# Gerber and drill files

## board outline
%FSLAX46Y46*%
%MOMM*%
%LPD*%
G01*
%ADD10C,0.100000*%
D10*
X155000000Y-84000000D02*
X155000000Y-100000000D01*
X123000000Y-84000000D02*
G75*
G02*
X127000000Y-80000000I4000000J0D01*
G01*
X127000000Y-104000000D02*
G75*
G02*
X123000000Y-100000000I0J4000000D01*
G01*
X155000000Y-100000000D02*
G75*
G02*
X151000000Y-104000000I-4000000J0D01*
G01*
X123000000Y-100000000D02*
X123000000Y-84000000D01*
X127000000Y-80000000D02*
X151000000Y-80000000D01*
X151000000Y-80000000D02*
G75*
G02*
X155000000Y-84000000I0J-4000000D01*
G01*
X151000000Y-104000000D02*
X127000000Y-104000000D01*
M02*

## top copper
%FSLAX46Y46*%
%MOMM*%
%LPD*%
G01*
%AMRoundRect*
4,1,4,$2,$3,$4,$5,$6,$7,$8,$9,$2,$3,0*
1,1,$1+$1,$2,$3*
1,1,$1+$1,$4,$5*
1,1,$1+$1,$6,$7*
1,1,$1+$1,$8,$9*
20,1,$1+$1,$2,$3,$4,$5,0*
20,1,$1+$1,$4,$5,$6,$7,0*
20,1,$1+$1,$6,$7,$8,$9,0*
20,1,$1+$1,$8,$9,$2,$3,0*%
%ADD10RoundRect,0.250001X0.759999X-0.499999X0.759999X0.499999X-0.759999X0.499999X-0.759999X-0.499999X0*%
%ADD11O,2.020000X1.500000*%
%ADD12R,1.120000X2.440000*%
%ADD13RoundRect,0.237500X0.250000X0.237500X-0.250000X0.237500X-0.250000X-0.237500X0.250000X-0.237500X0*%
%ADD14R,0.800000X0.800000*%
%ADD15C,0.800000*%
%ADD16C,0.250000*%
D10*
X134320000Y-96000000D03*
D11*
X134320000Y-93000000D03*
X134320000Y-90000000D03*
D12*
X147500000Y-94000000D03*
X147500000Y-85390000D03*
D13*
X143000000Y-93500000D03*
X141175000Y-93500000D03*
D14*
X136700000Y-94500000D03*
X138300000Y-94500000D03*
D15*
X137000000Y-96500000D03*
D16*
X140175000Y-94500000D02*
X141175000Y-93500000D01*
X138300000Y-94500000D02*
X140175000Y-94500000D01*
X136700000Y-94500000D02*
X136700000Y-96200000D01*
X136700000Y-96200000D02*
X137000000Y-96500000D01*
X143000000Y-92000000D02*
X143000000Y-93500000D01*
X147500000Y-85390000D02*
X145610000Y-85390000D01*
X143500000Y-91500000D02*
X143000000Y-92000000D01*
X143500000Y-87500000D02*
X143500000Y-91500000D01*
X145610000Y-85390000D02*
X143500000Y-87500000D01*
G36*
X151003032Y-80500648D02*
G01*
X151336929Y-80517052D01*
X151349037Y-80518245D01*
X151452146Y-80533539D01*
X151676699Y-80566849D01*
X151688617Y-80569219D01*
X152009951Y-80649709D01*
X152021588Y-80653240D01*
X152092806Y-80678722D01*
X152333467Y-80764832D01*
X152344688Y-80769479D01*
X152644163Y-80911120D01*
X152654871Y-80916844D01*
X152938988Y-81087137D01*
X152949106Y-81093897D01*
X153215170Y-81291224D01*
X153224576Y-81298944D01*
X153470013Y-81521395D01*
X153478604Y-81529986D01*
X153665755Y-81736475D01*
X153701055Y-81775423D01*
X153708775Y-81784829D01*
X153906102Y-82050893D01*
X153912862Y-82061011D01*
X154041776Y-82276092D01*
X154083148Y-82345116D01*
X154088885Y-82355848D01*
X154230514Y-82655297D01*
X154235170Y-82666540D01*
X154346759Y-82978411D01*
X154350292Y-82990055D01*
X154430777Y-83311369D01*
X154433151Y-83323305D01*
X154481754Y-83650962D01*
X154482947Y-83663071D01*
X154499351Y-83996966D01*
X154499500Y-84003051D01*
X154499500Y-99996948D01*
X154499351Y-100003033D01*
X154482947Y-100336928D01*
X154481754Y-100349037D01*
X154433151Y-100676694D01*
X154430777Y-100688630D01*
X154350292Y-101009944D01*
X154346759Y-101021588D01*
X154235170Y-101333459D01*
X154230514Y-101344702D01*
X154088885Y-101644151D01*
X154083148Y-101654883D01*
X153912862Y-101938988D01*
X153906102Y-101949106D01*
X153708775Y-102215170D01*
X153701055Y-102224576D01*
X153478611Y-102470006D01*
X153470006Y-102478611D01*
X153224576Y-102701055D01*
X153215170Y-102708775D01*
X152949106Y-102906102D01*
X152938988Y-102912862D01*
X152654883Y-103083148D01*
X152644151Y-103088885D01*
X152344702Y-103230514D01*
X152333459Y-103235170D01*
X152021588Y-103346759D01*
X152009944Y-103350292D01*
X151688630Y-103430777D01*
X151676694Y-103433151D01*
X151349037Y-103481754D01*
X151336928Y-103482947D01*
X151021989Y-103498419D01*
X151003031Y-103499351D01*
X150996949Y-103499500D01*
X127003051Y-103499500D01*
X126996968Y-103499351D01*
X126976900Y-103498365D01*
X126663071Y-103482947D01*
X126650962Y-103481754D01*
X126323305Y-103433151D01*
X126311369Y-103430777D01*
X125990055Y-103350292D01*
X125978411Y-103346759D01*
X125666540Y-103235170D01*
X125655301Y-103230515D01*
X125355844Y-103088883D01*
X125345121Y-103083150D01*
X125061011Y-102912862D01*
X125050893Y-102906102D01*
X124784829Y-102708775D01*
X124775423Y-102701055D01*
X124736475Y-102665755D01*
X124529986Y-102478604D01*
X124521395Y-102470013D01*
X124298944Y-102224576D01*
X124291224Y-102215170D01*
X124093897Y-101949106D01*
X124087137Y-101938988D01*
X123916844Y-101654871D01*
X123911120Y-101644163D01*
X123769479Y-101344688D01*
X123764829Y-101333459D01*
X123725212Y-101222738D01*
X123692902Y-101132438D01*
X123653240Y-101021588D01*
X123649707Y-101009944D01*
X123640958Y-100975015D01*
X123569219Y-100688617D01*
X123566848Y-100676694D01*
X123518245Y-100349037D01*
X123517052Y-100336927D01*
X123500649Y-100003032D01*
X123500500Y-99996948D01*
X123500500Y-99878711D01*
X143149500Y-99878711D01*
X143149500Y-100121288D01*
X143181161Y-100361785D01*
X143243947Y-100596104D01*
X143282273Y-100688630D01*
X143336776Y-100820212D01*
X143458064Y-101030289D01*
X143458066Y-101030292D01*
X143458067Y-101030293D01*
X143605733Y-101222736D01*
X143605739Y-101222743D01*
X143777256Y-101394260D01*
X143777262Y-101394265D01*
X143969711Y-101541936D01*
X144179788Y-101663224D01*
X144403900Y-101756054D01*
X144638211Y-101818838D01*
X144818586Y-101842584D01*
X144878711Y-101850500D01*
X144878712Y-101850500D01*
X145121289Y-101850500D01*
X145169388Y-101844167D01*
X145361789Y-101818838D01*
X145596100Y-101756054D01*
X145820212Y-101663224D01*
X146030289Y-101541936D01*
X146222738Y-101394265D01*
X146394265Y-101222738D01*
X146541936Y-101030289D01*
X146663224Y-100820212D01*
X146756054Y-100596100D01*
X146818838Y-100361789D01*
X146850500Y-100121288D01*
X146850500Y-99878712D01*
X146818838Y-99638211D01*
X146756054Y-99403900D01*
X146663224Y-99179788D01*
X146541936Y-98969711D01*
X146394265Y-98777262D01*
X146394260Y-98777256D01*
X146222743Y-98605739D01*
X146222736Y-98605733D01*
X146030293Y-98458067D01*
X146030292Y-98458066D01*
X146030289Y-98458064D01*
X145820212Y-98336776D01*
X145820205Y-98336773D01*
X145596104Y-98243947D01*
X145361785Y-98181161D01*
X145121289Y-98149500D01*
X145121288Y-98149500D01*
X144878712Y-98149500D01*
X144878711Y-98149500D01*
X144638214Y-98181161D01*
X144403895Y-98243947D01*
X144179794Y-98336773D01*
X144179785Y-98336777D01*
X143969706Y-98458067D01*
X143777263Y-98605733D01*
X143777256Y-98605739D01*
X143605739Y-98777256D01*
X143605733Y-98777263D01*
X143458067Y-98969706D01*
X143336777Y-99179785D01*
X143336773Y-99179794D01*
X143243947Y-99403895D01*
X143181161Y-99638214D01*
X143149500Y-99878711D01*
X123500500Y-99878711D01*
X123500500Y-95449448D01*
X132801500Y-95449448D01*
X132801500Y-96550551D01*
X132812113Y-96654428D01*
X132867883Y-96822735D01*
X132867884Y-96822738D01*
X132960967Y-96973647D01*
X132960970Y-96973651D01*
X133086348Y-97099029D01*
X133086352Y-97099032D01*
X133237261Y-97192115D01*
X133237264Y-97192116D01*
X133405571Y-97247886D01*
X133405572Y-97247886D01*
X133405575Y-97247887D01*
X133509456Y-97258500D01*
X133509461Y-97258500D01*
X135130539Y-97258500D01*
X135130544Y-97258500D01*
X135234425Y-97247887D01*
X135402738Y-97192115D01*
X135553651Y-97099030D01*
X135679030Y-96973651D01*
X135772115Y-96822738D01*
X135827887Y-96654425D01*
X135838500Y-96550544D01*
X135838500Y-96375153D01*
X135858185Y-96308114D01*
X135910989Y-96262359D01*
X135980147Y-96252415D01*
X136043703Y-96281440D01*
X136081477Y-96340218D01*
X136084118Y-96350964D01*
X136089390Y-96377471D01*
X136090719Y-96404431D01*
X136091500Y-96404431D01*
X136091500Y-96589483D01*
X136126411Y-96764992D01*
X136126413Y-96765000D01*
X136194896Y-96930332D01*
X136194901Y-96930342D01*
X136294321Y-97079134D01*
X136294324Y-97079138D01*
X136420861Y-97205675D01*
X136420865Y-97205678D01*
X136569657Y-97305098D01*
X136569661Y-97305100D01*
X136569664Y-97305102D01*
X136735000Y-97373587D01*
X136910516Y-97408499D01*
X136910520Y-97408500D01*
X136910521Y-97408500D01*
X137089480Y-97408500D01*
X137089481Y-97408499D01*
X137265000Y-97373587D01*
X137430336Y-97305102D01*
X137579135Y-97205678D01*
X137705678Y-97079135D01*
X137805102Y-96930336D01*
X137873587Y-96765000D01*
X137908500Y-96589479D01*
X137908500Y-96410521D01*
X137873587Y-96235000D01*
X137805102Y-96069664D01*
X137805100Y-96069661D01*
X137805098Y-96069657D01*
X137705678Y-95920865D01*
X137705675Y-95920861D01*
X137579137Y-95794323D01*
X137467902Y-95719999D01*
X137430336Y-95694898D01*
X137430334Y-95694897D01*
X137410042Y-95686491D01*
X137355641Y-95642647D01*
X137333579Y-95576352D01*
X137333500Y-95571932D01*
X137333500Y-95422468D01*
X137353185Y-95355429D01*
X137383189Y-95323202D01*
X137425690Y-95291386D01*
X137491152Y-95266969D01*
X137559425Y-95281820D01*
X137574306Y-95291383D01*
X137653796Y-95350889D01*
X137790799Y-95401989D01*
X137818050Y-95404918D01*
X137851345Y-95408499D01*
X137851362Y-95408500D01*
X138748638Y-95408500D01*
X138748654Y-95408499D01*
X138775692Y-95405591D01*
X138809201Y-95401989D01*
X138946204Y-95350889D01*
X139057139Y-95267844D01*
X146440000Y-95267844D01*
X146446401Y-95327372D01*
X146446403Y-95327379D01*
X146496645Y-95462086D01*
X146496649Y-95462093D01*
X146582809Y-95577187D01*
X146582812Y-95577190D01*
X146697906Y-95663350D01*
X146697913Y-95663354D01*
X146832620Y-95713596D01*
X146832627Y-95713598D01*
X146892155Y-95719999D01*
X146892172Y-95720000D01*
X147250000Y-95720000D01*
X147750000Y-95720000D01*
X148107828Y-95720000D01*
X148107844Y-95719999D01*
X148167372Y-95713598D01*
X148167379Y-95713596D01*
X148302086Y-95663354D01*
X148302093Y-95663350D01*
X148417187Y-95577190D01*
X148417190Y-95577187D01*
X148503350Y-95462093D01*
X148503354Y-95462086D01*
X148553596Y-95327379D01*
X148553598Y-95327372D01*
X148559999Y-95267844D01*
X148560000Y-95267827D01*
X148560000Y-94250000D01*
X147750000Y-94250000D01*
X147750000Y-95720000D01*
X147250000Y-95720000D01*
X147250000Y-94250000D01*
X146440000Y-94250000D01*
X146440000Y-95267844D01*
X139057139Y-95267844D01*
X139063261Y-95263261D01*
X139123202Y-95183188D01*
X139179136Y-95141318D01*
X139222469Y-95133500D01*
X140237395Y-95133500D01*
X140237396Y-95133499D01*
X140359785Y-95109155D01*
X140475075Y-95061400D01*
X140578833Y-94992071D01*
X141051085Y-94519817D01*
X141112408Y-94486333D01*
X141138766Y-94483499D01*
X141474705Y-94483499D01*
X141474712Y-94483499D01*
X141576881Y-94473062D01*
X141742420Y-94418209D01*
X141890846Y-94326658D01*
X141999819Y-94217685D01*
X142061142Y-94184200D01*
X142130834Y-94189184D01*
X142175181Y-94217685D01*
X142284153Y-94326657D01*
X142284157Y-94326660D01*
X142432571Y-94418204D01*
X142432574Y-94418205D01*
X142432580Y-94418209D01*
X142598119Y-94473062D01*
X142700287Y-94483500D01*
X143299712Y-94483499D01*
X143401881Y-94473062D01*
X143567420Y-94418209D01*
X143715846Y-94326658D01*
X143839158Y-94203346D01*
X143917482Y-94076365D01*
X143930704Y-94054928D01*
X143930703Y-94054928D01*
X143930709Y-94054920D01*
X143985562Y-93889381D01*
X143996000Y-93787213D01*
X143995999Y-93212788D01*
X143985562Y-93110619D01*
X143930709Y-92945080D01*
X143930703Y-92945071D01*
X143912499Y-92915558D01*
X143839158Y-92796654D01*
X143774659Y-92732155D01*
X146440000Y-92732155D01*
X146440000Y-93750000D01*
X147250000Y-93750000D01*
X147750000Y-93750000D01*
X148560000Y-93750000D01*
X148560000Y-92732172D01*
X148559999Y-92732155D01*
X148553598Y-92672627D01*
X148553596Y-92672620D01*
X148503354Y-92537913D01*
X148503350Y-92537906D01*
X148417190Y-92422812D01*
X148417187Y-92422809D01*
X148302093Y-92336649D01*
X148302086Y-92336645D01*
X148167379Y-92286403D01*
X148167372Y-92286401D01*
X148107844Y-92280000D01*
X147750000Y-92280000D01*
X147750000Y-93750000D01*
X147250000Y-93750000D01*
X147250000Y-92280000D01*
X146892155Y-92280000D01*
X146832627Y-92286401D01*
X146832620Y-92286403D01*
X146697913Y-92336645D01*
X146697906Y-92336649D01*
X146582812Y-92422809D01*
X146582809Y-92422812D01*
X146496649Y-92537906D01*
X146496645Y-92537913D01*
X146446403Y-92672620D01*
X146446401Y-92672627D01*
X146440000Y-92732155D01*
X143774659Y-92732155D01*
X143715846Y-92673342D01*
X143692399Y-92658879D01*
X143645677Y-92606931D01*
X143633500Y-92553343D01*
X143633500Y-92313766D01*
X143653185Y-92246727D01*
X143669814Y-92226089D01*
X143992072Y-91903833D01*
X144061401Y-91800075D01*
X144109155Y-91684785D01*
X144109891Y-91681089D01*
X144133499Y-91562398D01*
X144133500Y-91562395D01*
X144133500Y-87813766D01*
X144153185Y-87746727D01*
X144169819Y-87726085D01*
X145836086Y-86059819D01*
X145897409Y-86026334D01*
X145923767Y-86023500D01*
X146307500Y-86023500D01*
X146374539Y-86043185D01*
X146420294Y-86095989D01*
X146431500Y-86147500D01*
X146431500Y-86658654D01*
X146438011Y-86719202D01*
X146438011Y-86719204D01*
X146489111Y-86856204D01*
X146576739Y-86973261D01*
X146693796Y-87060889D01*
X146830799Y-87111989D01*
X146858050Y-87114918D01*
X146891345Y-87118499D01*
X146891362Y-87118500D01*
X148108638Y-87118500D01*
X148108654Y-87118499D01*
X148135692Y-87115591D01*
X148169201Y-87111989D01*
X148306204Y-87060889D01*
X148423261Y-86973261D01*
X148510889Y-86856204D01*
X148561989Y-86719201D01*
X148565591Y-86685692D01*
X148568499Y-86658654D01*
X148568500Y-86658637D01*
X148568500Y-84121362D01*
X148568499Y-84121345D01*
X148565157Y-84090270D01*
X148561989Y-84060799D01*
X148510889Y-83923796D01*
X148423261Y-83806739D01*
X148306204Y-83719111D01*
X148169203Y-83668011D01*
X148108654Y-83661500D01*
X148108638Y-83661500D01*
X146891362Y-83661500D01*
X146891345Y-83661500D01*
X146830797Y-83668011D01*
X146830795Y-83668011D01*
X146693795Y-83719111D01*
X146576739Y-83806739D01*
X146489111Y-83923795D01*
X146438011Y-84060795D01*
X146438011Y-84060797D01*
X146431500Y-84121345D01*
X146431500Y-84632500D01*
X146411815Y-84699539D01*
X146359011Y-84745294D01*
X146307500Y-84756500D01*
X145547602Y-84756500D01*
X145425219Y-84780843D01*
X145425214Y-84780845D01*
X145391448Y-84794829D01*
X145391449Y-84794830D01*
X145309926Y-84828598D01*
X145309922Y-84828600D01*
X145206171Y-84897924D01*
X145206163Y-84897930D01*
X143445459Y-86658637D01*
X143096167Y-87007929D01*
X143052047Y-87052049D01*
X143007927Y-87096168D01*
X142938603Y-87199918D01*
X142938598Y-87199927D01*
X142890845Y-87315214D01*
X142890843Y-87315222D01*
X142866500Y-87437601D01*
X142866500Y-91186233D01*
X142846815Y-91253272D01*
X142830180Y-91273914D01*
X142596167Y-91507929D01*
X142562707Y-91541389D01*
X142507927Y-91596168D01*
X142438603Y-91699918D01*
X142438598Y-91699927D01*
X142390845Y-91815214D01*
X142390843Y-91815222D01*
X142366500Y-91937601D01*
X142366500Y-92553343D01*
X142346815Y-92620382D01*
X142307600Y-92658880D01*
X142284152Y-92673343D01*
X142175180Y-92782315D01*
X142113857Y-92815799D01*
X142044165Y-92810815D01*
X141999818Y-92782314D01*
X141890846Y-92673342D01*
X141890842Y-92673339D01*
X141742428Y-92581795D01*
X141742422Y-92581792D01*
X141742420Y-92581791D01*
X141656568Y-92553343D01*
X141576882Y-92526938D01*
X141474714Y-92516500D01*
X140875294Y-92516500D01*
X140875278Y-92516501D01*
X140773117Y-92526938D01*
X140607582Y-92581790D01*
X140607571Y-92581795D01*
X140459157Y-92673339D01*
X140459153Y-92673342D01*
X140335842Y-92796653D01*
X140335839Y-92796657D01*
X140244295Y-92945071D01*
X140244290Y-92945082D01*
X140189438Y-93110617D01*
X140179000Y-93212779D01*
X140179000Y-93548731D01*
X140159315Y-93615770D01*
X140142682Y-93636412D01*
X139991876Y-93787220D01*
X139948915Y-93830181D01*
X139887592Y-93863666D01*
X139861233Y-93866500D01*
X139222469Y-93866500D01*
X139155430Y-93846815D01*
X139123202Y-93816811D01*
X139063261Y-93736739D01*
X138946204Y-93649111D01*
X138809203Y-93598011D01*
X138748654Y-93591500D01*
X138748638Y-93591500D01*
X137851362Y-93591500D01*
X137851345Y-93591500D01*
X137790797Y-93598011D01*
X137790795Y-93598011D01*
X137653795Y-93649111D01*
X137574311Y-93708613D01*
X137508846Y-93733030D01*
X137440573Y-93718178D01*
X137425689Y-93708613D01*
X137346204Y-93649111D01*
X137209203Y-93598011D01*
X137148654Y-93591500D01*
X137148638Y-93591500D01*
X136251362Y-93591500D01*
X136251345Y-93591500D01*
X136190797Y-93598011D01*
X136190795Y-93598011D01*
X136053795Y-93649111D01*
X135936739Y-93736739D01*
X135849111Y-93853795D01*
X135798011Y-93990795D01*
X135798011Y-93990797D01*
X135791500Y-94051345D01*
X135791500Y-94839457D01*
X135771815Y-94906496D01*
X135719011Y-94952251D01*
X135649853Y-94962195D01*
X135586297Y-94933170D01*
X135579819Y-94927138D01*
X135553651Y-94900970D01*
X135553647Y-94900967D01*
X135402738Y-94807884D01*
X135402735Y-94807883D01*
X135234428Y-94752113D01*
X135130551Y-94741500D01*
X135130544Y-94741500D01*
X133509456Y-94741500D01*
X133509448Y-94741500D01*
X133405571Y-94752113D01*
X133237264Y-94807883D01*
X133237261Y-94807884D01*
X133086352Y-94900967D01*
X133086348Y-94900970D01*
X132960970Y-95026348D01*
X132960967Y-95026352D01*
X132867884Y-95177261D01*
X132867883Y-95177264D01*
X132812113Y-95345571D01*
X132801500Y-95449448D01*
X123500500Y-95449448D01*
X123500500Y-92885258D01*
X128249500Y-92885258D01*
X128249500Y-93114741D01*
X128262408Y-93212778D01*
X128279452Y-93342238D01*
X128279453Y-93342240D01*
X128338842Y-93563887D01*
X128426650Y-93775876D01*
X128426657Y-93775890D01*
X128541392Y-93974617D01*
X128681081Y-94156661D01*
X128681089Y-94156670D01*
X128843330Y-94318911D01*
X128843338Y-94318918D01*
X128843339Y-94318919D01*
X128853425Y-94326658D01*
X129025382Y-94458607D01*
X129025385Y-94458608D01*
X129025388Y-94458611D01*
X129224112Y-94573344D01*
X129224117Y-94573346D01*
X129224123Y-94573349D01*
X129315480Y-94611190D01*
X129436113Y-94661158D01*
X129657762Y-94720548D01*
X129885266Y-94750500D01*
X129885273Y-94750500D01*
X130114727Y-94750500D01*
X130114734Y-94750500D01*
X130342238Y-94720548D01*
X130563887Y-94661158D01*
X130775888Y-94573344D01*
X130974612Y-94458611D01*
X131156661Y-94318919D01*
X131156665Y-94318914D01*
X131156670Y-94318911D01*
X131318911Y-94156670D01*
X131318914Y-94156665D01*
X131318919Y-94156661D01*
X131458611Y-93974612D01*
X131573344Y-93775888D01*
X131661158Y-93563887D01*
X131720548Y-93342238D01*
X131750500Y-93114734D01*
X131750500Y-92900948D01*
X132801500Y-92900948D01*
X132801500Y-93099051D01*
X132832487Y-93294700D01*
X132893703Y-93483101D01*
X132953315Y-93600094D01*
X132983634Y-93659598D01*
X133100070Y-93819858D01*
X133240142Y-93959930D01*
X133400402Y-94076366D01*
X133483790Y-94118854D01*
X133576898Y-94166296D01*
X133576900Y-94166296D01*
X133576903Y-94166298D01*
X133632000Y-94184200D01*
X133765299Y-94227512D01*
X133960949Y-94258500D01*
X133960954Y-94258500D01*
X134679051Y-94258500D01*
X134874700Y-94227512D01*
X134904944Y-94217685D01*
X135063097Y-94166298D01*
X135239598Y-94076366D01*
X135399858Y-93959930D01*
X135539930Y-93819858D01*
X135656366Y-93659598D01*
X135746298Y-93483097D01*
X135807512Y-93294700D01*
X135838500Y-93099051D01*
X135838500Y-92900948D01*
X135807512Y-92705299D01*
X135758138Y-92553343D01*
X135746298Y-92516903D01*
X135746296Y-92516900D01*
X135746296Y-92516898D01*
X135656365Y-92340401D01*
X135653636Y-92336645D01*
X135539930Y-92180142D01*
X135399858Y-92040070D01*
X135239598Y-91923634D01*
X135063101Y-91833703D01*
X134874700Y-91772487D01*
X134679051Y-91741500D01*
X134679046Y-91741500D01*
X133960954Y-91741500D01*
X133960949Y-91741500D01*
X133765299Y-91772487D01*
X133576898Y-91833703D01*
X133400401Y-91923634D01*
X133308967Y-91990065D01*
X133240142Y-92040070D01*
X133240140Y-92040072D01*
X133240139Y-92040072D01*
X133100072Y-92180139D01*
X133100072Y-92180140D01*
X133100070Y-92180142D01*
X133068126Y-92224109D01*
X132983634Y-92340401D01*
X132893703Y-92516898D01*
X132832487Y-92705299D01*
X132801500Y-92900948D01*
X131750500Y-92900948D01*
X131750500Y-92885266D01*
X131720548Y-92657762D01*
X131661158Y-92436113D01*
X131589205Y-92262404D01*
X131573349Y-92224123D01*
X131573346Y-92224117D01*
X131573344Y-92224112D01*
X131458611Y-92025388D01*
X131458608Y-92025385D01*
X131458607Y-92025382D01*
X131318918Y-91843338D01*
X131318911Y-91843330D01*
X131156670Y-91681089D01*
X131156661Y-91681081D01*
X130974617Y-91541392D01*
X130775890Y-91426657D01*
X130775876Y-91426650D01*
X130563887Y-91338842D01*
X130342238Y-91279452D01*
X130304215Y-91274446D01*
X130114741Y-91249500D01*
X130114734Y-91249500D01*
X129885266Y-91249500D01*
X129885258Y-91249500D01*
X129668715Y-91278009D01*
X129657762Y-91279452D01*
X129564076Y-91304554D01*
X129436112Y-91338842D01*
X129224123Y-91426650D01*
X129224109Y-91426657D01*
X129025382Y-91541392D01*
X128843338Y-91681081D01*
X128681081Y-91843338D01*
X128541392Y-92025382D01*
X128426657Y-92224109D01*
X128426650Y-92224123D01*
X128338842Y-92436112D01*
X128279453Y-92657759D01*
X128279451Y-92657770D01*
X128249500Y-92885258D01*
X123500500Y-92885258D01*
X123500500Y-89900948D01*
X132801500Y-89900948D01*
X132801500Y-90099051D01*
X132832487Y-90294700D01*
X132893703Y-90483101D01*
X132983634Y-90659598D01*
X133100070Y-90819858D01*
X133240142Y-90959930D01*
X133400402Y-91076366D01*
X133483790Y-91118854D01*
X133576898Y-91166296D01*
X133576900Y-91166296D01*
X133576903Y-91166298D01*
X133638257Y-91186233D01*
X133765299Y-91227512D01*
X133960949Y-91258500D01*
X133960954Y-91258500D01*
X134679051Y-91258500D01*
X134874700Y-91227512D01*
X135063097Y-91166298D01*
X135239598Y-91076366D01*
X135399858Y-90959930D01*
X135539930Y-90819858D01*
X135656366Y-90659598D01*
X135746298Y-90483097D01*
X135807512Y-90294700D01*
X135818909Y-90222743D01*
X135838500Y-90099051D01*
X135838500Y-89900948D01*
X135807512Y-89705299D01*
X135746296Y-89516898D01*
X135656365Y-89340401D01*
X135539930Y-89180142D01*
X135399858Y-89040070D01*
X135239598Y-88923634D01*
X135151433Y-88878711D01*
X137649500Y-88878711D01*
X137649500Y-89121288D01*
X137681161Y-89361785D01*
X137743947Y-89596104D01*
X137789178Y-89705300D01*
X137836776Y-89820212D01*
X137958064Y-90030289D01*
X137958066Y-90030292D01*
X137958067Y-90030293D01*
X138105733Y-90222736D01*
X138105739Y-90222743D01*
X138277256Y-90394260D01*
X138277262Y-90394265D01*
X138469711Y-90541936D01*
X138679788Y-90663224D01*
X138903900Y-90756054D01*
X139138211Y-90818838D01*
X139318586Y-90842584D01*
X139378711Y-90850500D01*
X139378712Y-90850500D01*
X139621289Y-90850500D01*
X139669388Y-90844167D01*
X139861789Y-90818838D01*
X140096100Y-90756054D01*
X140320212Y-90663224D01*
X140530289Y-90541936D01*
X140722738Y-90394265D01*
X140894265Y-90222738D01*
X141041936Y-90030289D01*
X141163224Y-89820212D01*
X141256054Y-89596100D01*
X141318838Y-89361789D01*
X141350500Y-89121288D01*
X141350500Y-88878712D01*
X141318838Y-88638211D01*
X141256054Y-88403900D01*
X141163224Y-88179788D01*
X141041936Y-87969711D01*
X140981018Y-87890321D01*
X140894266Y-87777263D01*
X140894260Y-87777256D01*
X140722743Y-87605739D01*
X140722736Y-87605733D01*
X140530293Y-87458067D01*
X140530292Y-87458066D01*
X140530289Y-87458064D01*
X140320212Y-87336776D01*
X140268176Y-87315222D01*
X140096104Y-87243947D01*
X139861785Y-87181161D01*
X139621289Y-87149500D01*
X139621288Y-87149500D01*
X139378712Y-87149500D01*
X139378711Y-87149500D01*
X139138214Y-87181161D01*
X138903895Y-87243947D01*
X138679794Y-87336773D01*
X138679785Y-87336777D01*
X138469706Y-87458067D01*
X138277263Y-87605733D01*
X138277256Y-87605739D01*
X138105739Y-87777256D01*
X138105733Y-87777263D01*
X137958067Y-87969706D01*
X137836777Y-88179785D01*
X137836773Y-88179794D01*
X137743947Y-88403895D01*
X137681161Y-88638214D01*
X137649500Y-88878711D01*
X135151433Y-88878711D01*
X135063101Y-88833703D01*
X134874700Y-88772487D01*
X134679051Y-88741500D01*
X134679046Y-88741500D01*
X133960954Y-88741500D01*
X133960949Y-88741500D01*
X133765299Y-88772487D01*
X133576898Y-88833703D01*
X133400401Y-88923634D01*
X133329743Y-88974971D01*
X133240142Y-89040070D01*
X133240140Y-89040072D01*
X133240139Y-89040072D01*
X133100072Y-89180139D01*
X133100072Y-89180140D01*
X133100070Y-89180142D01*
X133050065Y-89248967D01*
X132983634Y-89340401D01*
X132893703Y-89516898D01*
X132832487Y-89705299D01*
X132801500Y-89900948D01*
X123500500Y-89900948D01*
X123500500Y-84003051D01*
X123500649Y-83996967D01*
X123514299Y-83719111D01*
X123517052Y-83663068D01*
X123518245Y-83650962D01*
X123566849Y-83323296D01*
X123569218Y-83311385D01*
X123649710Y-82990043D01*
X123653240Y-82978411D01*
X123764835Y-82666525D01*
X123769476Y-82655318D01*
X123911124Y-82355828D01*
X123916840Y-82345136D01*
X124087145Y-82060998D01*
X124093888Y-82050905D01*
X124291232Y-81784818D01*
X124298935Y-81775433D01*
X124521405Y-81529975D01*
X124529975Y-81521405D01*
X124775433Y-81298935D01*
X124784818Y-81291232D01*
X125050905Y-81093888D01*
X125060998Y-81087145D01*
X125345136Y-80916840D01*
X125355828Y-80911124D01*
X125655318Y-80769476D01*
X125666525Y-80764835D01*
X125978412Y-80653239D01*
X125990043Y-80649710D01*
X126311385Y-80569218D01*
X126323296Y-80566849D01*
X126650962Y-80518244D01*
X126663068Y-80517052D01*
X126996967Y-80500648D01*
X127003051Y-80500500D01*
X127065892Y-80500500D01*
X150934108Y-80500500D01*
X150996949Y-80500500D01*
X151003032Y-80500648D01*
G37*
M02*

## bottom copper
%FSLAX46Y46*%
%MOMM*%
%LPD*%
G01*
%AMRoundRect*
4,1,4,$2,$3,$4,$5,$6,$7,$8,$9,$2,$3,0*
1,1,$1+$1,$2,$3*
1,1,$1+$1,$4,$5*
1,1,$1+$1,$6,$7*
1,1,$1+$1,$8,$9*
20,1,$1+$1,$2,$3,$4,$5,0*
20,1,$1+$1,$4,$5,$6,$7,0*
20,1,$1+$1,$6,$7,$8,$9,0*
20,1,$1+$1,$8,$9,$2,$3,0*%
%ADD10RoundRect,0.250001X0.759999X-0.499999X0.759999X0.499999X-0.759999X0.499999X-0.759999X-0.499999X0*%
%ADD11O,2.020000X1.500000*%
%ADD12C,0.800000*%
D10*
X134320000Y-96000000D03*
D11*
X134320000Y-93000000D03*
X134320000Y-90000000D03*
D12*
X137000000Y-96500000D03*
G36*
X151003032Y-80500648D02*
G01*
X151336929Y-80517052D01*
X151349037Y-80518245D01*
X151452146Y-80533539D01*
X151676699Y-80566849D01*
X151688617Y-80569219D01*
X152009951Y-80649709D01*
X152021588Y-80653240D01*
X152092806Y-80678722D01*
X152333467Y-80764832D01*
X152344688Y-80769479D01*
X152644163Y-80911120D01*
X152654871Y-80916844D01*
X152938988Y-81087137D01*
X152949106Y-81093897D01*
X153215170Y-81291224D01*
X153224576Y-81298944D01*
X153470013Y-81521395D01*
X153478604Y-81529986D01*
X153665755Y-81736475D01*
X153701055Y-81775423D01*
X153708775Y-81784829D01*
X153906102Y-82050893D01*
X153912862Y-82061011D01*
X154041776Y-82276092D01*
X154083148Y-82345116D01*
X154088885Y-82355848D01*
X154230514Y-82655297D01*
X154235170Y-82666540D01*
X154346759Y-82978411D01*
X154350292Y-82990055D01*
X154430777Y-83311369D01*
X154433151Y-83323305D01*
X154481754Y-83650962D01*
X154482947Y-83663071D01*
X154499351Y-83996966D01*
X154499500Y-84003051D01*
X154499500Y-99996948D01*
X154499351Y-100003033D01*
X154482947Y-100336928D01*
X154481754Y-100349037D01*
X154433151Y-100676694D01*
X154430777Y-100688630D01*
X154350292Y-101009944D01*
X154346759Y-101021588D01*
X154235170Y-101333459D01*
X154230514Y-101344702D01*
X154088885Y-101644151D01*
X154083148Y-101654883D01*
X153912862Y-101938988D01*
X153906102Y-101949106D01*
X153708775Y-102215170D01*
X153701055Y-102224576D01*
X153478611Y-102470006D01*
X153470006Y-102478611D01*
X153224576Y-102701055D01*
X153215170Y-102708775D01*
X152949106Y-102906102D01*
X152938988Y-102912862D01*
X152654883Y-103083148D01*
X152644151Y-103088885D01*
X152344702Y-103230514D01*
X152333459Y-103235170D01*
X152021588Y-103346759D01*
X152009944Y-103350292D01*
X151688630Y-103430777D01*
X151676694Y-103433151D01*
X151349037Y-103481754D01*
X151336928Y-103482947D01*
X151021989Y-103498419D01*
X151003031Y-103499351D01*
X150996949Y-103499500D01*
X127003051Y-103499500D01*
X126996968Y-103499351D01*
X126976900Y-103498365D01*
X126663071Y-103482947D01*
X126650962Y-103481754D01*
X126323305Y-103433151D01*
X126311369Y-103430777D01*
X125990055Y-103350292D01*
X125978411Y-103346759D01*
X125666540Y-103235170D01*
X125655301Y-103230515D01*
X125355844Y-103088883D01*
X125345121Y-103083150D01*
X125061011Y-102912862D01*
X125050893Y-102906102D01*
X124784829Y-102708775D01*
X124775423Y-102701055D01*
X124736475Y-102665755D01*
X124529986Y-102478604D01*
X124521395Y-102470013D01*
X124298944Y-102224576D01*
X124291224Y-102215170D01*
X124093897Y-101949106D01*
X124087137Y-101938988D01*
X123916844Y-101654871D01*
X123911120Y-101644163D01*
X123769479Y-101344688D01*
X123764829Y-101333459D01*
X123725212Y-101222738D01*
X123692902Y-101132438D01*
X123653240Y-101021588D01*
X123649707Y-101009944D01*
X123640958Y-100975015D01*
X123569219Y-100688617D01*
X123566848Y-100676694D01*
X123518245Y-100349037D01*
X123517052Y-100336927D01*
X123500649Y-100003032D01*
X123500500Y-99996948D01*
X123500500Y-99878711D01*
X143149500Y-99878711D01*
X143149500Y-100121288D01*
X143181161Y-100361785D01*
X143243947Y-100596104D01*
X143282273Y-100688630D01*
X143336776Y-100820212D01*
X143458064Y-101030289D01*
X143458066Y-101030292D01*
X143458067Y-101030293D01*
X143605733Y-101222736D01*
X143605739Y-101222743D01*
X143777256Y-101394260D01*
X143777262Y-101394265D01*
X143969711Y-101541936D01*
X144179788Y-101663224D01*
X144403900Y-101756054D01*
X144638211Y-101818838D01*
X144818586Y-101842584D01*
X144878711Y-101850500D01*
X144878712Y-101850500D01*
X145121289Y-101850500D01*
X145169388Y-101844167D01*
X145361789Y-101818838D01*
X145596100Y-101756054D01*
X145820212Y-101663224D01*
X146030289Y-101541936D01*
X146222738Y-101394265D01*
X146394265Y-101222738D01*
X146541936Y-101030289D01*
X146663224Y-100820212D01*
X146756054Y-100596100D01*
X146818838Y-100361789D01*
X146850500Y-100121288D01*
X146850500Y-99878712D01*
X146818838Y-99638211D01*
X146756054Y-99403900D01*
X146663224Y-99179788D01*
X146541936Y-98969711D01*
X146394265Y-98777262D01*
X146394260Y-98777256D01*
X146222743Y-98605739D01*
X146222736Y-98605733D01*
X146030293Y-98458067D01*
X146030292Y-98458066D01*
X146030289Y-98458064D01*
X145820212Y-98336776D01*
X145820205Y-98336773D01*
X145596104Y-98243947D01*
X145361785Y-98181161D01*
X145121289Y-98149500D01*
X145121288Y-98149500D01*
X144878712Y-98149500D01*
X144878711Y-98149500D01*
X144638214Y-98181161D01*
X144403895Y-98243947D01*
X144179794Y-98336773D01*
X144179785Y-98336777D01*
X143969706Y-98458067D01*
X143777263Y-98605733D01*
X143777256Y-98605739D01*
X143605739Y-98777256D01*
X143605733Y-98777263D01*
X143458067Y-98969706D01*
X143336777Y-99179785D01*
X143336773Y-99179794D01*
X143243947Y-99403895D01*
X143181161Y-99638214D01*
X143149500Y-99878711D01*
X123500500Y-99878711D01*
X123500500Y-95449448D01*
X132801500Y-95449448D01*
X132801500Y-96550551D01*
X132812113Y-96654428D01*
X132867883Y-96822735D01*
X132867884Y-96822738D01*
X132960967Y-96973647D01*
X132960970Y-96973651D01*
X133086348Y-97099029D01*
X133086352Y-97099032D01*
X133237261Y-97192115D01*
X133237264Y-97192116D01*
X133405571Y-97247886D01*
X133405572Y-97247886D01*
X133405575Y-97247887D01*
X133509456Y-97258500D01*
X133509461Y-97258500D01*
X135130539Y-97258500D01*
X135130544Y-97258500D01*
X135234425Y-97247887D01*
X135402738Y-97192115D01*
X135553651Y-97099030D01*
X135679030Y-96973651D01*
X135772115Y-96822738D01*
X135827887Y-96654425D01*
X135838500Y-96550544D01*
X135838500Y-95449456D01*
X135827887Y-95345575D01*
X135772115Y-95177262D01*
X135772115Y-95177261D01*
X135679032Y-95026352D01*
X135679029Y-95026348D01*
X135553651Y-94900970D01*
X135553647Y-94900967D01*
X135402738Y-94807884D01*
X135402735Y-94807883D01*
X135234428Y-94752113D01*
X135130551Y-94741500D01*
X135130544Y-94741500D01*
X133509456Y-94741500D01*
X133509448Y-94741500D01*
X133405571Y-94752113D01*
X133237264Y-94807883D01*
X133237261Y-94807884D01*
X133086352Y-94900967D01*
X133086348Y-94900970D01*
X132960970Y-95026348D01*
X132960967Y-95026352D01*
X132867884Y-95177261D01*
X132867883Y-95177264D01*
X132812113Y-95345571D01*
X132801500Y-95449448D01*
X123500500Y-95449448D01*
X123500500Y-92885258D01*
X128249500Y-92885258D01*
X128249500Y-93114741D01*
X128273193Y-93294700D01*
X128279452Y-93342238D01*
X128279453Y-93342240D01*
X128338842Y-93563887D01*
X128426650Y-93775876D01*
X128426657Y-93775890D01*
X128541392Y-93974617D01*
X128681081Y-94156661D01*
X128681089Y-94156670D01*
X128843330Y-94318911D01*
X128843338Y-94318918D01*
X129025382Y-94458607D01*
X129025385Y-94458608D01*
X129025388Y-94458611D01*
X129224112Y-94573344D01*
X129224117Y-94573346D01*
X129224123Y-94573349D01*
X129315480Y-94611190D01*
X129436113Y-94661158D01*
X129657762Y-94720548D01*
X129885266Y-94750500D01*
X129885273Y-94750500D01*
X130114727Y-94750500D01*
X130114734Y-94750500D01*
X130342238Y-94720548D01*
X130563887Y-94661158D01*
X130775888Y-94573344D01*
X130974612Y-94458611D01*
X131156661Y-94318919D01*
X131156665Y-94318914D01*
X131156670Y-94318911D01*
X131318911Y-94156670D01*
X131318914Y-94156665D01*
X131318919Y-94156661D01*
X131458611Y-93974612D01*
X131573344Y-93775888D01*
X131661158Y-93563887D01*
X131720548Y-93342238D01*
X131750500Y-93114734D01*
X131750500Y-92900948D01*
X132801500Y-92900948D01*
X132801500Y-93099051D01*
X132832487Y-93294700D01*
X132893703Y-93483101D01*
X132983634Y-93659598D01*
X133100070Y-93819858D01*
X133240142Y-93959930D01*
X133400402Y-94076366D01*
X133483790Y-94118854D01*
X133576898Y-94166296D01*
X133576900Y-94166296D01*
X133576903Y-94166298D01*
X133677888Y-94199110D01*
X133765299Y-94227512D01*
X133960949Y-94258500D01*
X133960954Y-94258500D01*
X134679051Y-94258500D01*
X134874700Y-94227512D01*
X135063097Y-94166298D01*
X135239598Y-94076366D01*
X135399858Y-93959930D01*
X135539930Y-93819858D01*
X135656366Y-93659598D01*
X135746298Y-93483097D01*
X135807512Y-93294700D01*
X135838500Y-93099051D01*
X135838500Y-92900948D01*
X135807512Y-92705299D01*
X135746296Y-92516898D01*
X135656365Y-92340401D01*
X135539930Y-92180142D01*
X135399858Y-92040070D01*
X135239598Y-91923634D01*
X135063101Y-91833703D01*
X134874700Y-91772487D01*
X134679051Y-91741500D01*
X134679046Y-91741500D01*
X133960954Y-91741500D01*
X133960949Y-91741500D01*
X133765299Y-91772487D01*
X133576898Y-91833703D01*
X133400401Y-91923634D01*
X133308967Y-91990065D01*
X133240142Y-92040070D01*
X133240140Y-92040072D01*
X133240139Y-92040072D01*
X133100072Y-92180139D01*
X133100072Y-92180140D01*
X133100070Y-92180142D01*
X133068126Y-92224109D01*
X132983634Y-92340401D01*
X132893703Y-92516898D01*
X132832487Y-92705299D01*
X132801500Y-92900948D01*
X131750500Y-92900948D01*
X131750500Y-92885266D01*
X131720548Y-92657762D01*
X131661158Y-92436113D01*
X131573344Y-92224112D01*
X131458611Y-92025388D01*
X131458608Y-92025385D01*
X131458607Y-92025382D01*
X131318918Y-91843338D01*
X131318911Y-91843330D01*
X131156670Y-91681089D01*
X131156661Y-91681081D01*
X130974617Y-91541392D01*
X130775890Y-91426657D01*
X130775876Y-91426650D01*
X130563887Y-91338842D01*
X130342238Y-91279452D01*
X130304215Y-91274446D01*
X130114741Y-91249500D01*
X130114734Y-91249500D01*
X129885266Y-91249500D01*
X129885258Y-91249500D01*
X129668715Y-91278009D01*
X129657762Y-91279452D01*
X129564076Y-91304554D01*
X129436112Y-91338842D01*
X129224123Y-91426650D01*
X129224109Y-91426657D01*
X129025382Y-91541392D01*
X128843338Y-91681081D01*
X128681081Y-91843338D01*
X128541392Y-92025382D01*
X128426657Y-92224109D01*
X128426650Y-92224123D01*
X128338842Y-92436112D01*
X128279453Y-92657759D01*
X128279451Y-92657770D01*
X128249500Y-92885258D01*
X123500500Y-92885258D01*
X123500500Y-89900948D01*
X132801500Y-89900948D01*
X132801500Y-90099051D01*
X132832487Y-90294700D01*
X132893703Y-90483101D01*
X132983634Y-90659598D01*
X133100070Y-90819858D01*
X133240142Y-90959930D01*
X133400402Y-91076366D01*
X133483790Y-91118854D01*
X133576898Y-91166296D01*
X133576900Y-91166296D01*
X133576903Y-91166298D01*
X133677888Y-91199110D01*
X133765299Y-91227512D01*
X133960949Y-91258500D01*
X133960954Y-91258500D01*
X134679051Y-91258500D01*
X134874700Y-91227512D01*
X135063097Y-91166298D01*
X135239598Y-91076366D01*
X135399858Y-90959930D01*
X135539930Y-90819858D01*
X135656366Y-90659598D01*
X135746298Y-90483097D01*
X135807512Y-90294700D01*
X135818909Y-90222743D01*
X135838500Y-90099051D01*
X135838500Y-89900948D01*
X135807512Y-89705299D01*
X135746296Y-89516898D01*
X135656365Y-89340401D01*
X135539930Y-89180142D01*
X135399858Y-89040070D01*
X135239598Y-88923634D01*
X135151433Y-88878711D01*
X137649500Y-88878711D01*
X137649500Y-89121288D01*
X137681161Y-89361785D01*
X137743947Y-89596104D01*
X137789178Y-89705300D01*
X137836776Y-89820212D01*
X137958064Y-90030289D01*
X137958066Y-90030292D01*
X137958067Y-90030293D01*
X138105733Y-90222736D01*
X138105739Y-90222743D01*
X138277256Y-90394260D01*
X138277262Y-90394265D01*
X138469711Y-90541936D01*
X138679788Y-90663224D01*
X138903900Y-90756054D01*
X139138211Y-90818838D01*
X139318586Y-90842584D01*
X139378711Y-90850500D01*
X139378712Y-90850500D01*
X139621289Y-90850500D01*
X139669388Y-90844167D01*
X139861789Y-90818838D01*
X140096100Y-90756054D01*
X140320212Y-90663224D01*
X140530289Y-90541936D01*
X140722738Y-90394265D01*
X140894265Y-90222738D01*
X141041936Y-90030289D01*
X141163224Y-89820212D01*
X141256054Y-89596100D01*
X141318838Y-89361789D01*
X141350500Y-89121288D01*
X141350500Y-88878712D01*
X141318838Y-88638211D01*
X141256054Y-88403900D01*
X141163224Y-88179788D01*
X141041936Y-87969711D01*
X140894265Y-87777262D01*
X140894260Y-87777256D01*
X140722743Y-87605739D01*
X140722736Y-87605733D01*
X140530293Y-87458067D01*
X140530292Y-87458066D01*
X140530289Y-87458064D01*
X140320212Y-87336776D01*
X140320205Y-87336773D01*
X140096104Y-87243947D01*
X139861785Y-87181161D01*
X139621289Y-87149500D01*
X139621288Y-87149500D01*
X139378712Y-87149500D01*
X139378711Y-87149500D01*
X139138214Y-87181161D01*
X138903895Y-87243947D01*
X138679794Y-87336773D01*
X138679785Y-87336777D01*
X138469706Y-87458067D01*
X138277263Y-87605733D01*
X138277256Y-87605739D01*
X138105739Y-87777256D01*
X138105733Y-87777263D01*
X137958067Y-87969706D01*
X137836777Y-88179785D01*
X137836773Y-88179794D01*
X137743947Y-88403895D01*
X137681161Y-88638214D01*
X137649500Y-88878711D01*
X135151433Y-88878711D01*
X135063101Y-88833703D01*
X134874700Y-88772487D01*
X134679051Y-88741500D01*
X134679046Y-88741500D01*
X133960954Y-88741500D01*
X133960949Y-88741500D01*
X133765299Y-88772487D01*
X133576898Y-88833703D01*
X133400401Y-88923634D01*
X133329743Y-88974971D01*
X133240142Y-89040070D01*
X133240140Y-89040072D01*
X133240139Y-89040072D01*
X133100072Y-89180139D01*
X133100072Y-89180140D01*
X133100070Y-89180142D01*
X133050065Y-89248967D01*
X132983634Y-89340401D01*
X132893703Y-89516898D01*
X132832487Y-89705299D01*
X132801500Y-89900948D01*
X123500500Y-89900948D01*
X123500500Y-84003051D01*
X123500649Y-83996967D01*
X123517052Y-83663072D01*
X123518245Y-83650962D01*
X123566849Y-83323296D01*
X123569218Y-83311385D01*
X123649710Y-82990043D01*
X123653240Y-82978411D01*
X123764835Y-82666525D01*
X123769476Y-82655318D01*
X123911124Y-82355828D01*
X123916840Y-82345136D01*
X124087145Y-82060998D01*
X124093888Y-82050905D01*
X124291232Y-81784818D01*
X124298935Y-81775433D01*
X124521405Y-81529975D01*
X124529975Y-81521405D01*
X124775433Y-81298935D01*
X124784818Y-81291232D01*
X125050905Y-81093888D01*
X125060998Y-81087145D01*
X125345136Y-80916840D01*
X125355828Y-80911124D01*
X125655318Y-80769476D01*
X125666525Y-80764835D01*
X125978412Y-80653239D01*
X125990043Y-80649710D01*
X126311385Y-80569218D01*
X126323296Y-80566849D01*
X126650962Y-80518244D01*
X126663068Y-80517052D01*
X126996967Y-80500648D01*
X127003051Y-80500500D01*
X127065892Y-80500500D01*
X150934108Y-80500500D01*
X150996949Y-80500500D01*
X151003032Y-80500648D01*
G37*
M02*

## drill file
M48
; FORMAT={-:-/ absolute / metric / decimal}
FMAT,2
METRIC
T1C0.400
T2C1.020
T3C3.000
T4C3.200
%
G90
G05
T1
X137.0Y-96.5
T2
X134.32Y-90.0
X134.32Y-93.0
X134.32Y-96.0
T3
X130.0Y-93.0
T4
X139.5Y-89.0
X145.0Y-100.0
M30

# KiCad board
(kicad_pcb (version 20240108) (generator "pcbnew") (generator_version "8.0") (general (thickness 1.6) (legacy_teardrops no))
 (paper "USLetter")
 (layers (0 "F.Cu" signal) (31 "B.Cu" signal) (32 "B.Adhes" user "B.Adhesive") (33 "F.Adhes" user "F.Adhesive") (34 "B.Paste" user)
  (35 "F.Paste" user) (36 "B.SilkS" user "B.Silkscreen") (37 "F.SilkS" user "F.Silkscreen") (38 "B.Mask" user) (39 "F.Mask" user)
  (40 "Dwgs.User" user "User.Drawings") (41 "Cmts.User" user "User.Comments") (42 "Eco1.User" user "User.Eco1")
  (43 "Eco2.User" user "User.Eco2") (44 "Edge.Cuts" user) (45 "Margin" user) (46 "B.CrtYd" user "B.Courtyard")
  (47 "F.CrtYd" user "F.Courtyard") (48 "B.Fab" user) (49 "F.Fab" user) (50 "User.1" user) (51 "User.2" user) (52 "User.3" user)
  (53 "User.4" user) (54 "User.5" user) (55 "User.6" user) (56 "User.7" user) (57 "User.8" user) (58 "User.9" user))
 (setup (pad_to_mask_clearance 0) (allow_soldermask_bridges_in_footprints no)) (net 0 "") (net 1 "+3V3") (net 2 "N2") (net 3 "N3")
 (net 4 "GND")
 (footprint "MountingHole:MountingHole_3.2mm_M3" (layer "F.Cu") (at 139.5 89)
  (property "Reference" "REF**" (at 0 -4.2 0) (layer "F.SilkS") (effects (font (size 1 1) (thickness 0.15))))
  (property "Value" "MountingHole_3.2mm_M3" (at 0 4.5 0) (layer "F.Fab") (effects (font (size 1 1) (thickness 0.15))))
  (pad "" np_thru_hole circle (at 0 0) (size 3.2 3.2) (drill 3.2) (layers "*.Cu" "*.Mask")))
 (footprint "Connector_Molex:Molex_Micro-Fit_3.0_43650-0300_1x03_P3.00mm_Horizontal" (layer "F.Cu") (at 134.32 96 90)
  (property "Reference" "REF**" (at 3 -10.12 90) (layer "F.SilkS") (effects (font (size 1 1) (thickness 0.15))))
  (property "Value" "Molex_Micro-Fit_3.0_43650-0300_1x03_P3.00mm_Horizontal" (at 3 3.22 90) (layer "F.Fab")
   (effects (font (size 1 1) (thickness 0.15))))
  (pad "" np_thru_hole circle (at 3 -4.32 90) (size 3 3) (drill 3) (layers "*.Cu" "*.Mask"))
  (pad "1" thru_hole roundrect (at 0 0 90) (size 1.5 2.02) (drill 1.02) (layers "*.Cu" "*.Mask") (remove_unused_layers no)
   (roundrect_rratio 0.166667))
  (pad "2" thru_hole oval (at 3 0 90) (size 1.5 2.02) (drill 1.02) (layers "*.Cu" "*.Mask") (remove_unused_layers no))
  (pad "3" thru_hole oval (at 6 0 90) (size 1.5 2.02) (drill 1.02) (layers "*.Cu" "*.Mask") (remove_unused_layers no)))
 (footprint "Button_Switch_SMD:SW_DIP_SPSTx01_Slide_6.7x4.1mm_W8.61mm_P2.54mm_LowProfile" (layer "F.Cu") (at 147.5 89.695 90)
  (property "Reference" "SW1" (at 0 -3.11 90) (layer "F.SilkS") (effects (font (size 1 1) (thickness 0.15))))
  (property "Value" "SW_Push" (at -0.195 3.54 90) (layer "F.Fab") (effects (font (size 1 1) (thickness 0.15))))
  (pad "1" smd rect (at -4.305 0 90) (size 2.44 1.12) (layers "F.Cu" "F.Paste" "F.Mask") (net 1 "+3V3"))
  (pad "2" smd rect (at 4.305 0 90) (size 2.44 1.12) (layers "F.Cu" "F.Paste" "F.Mask") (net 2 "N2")))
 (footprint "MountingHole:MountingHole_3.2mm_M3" (layer "F.Cu") (at 145 100)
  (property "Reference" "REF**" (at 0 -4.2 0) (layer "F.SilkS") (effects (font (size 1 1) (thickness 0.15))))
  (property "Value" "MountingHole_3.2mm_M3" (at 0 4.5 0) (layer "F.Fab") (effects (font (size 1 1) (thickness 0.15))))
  (pad "" np_thru_hole circle (at 0 0) (size 3.2 3.2) (drill 3.2) (layers "*.Cu" "*.Mask")))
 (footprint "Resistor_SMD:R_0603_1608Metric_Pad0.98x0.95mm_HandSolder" (layer "F.Cu") (at 142.0875 93.5 180)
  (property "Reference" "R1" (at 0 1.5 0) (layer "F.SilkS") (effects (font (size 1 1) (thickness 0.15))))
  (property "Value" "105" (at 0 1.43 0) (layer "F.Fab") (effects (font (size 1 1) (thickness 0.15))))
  (pad "1" smd roundrect (at -0.9125 0 180) (size 0.975 0.95) (layers "F.Cu" "F.Paste" "F.Mask") (roundrect_rratio 0.25) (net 2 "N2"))
  (pad "2" smd roundrect (at 0.9125 0 180) (size 0.975 0.95) (layers "F.Cu" "F.Paste" "F.Mask") (roundrect_rratio 0.25) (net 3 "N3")))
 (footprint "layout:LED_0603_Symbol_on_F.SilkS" (layer "F.Cu") (at 137.5 94.5)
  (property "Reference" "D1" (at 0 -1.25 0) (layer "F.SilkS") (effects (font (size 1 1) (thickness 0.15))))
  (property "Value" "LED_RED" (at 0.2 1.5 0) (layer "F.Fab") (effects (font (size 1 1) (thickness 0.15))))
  (pad "1" smd rect (at -0.8 0 180) (size 0.8 0.8) (layers "F.Cu" "F.Paste" "F.Mask") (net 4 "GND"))
  (pad "2" smd rect (at 0.8 0 180) (size 0.8 0.8) (layers "F.Cu" "F.Paste" "F.Mask") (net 3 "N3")))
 (gr_line (start 155 84) (end 155 100) (stroke (width 0.1) (type default)) (layer "Edge.Cuts"))
 (gr_arc (start 123 84) (mid 124.171573 81.171573) (end 127 80) (stroke (width 0.1) (type default)) (layer "Edge.Cuts"))
 (gr_arc (start 127 104) (mid 124.171573 102.828427) (end 123 100) (stroke (width 0.1) (type default)) (layer "Edge.Cuts"))
 (gr_arc (start 155 100) (mid 153.828427 102.828427) (end 151 104) (stroke (width 0.1) (type default)) (layer "Edge.Cuts"))
 (gr_line (start 123 100) (end 123 84) (stroke (width 0.1) (type default)) (layer "Edge.Cuts"))
 (gr_line (start 127 80) (end 151 80) (stroke (width 0.1) (type default)) (layer "Edge.Cuts"))
 (gr_arc (start 151 80) (mid 153.828427 81.171573) (end 155 84) (stroke (width 0.1) (type default)) (layer "Edge.Cuts"))
 (gr_line (start 151 104) (end 127 104) (stroke (width 0.1) (type default)) (layer "Edge.Cuts"))
 (segment (start 140.175 94.5) (end 141.175 93.5) (width 0.25) (layer "F.Cu") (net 3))
 (segment (start 138.3 94.5) (end 140.175 94.5) (width 0.25) (layer "F.Cu") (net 3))
 (segment (start 136.7 94.5) (end 136.7 96.2) (width 0.25) (layer "F.Cu") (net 4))
 (segment (start 136.7 96.2) (end 137 96.5) (width 0.25) (layer "F.Cu") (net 4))
 (via (at 137 96.5) (size 0.8) (drill 0.4) (layers "F.Cu" "B.Cu") (free yes) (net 4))
 (segment (start 143 92) (end 143 93.5) (width 0.25) (layer "F.Cu") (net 2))
 (segment (start 147.5 85.39) (end 145.61 85.39) (width 0.25) (layer "F.Cu") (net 2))
 (segment (start 143.5 91.5) (end 143 92) (width 0.25) (layer "F.Cu") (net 2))
 (segment (start 143.5 87.5) (end 143.5 91.5) (width 0.25) (layer "F.Cu") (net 2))
 (segment (start 145.61 85.39) (end 143.5 87.5) (width 0.25) (layer "F.Cu") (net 2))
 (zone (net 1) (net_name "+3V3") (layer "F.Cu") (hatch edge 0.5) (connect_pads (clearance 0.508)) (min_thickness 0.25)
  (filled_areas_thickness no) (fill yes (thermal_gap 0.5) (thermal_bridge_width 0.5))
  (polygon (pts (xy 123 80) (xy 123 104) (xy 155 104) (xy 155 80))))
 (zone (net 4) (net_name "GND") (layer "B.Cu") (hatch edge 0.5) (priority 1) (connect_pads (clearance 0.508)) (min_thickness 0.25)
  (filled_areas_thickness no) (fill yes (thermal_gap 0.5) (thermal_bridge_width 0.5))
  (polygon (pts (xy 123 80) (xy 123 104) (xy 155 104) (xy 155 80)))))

